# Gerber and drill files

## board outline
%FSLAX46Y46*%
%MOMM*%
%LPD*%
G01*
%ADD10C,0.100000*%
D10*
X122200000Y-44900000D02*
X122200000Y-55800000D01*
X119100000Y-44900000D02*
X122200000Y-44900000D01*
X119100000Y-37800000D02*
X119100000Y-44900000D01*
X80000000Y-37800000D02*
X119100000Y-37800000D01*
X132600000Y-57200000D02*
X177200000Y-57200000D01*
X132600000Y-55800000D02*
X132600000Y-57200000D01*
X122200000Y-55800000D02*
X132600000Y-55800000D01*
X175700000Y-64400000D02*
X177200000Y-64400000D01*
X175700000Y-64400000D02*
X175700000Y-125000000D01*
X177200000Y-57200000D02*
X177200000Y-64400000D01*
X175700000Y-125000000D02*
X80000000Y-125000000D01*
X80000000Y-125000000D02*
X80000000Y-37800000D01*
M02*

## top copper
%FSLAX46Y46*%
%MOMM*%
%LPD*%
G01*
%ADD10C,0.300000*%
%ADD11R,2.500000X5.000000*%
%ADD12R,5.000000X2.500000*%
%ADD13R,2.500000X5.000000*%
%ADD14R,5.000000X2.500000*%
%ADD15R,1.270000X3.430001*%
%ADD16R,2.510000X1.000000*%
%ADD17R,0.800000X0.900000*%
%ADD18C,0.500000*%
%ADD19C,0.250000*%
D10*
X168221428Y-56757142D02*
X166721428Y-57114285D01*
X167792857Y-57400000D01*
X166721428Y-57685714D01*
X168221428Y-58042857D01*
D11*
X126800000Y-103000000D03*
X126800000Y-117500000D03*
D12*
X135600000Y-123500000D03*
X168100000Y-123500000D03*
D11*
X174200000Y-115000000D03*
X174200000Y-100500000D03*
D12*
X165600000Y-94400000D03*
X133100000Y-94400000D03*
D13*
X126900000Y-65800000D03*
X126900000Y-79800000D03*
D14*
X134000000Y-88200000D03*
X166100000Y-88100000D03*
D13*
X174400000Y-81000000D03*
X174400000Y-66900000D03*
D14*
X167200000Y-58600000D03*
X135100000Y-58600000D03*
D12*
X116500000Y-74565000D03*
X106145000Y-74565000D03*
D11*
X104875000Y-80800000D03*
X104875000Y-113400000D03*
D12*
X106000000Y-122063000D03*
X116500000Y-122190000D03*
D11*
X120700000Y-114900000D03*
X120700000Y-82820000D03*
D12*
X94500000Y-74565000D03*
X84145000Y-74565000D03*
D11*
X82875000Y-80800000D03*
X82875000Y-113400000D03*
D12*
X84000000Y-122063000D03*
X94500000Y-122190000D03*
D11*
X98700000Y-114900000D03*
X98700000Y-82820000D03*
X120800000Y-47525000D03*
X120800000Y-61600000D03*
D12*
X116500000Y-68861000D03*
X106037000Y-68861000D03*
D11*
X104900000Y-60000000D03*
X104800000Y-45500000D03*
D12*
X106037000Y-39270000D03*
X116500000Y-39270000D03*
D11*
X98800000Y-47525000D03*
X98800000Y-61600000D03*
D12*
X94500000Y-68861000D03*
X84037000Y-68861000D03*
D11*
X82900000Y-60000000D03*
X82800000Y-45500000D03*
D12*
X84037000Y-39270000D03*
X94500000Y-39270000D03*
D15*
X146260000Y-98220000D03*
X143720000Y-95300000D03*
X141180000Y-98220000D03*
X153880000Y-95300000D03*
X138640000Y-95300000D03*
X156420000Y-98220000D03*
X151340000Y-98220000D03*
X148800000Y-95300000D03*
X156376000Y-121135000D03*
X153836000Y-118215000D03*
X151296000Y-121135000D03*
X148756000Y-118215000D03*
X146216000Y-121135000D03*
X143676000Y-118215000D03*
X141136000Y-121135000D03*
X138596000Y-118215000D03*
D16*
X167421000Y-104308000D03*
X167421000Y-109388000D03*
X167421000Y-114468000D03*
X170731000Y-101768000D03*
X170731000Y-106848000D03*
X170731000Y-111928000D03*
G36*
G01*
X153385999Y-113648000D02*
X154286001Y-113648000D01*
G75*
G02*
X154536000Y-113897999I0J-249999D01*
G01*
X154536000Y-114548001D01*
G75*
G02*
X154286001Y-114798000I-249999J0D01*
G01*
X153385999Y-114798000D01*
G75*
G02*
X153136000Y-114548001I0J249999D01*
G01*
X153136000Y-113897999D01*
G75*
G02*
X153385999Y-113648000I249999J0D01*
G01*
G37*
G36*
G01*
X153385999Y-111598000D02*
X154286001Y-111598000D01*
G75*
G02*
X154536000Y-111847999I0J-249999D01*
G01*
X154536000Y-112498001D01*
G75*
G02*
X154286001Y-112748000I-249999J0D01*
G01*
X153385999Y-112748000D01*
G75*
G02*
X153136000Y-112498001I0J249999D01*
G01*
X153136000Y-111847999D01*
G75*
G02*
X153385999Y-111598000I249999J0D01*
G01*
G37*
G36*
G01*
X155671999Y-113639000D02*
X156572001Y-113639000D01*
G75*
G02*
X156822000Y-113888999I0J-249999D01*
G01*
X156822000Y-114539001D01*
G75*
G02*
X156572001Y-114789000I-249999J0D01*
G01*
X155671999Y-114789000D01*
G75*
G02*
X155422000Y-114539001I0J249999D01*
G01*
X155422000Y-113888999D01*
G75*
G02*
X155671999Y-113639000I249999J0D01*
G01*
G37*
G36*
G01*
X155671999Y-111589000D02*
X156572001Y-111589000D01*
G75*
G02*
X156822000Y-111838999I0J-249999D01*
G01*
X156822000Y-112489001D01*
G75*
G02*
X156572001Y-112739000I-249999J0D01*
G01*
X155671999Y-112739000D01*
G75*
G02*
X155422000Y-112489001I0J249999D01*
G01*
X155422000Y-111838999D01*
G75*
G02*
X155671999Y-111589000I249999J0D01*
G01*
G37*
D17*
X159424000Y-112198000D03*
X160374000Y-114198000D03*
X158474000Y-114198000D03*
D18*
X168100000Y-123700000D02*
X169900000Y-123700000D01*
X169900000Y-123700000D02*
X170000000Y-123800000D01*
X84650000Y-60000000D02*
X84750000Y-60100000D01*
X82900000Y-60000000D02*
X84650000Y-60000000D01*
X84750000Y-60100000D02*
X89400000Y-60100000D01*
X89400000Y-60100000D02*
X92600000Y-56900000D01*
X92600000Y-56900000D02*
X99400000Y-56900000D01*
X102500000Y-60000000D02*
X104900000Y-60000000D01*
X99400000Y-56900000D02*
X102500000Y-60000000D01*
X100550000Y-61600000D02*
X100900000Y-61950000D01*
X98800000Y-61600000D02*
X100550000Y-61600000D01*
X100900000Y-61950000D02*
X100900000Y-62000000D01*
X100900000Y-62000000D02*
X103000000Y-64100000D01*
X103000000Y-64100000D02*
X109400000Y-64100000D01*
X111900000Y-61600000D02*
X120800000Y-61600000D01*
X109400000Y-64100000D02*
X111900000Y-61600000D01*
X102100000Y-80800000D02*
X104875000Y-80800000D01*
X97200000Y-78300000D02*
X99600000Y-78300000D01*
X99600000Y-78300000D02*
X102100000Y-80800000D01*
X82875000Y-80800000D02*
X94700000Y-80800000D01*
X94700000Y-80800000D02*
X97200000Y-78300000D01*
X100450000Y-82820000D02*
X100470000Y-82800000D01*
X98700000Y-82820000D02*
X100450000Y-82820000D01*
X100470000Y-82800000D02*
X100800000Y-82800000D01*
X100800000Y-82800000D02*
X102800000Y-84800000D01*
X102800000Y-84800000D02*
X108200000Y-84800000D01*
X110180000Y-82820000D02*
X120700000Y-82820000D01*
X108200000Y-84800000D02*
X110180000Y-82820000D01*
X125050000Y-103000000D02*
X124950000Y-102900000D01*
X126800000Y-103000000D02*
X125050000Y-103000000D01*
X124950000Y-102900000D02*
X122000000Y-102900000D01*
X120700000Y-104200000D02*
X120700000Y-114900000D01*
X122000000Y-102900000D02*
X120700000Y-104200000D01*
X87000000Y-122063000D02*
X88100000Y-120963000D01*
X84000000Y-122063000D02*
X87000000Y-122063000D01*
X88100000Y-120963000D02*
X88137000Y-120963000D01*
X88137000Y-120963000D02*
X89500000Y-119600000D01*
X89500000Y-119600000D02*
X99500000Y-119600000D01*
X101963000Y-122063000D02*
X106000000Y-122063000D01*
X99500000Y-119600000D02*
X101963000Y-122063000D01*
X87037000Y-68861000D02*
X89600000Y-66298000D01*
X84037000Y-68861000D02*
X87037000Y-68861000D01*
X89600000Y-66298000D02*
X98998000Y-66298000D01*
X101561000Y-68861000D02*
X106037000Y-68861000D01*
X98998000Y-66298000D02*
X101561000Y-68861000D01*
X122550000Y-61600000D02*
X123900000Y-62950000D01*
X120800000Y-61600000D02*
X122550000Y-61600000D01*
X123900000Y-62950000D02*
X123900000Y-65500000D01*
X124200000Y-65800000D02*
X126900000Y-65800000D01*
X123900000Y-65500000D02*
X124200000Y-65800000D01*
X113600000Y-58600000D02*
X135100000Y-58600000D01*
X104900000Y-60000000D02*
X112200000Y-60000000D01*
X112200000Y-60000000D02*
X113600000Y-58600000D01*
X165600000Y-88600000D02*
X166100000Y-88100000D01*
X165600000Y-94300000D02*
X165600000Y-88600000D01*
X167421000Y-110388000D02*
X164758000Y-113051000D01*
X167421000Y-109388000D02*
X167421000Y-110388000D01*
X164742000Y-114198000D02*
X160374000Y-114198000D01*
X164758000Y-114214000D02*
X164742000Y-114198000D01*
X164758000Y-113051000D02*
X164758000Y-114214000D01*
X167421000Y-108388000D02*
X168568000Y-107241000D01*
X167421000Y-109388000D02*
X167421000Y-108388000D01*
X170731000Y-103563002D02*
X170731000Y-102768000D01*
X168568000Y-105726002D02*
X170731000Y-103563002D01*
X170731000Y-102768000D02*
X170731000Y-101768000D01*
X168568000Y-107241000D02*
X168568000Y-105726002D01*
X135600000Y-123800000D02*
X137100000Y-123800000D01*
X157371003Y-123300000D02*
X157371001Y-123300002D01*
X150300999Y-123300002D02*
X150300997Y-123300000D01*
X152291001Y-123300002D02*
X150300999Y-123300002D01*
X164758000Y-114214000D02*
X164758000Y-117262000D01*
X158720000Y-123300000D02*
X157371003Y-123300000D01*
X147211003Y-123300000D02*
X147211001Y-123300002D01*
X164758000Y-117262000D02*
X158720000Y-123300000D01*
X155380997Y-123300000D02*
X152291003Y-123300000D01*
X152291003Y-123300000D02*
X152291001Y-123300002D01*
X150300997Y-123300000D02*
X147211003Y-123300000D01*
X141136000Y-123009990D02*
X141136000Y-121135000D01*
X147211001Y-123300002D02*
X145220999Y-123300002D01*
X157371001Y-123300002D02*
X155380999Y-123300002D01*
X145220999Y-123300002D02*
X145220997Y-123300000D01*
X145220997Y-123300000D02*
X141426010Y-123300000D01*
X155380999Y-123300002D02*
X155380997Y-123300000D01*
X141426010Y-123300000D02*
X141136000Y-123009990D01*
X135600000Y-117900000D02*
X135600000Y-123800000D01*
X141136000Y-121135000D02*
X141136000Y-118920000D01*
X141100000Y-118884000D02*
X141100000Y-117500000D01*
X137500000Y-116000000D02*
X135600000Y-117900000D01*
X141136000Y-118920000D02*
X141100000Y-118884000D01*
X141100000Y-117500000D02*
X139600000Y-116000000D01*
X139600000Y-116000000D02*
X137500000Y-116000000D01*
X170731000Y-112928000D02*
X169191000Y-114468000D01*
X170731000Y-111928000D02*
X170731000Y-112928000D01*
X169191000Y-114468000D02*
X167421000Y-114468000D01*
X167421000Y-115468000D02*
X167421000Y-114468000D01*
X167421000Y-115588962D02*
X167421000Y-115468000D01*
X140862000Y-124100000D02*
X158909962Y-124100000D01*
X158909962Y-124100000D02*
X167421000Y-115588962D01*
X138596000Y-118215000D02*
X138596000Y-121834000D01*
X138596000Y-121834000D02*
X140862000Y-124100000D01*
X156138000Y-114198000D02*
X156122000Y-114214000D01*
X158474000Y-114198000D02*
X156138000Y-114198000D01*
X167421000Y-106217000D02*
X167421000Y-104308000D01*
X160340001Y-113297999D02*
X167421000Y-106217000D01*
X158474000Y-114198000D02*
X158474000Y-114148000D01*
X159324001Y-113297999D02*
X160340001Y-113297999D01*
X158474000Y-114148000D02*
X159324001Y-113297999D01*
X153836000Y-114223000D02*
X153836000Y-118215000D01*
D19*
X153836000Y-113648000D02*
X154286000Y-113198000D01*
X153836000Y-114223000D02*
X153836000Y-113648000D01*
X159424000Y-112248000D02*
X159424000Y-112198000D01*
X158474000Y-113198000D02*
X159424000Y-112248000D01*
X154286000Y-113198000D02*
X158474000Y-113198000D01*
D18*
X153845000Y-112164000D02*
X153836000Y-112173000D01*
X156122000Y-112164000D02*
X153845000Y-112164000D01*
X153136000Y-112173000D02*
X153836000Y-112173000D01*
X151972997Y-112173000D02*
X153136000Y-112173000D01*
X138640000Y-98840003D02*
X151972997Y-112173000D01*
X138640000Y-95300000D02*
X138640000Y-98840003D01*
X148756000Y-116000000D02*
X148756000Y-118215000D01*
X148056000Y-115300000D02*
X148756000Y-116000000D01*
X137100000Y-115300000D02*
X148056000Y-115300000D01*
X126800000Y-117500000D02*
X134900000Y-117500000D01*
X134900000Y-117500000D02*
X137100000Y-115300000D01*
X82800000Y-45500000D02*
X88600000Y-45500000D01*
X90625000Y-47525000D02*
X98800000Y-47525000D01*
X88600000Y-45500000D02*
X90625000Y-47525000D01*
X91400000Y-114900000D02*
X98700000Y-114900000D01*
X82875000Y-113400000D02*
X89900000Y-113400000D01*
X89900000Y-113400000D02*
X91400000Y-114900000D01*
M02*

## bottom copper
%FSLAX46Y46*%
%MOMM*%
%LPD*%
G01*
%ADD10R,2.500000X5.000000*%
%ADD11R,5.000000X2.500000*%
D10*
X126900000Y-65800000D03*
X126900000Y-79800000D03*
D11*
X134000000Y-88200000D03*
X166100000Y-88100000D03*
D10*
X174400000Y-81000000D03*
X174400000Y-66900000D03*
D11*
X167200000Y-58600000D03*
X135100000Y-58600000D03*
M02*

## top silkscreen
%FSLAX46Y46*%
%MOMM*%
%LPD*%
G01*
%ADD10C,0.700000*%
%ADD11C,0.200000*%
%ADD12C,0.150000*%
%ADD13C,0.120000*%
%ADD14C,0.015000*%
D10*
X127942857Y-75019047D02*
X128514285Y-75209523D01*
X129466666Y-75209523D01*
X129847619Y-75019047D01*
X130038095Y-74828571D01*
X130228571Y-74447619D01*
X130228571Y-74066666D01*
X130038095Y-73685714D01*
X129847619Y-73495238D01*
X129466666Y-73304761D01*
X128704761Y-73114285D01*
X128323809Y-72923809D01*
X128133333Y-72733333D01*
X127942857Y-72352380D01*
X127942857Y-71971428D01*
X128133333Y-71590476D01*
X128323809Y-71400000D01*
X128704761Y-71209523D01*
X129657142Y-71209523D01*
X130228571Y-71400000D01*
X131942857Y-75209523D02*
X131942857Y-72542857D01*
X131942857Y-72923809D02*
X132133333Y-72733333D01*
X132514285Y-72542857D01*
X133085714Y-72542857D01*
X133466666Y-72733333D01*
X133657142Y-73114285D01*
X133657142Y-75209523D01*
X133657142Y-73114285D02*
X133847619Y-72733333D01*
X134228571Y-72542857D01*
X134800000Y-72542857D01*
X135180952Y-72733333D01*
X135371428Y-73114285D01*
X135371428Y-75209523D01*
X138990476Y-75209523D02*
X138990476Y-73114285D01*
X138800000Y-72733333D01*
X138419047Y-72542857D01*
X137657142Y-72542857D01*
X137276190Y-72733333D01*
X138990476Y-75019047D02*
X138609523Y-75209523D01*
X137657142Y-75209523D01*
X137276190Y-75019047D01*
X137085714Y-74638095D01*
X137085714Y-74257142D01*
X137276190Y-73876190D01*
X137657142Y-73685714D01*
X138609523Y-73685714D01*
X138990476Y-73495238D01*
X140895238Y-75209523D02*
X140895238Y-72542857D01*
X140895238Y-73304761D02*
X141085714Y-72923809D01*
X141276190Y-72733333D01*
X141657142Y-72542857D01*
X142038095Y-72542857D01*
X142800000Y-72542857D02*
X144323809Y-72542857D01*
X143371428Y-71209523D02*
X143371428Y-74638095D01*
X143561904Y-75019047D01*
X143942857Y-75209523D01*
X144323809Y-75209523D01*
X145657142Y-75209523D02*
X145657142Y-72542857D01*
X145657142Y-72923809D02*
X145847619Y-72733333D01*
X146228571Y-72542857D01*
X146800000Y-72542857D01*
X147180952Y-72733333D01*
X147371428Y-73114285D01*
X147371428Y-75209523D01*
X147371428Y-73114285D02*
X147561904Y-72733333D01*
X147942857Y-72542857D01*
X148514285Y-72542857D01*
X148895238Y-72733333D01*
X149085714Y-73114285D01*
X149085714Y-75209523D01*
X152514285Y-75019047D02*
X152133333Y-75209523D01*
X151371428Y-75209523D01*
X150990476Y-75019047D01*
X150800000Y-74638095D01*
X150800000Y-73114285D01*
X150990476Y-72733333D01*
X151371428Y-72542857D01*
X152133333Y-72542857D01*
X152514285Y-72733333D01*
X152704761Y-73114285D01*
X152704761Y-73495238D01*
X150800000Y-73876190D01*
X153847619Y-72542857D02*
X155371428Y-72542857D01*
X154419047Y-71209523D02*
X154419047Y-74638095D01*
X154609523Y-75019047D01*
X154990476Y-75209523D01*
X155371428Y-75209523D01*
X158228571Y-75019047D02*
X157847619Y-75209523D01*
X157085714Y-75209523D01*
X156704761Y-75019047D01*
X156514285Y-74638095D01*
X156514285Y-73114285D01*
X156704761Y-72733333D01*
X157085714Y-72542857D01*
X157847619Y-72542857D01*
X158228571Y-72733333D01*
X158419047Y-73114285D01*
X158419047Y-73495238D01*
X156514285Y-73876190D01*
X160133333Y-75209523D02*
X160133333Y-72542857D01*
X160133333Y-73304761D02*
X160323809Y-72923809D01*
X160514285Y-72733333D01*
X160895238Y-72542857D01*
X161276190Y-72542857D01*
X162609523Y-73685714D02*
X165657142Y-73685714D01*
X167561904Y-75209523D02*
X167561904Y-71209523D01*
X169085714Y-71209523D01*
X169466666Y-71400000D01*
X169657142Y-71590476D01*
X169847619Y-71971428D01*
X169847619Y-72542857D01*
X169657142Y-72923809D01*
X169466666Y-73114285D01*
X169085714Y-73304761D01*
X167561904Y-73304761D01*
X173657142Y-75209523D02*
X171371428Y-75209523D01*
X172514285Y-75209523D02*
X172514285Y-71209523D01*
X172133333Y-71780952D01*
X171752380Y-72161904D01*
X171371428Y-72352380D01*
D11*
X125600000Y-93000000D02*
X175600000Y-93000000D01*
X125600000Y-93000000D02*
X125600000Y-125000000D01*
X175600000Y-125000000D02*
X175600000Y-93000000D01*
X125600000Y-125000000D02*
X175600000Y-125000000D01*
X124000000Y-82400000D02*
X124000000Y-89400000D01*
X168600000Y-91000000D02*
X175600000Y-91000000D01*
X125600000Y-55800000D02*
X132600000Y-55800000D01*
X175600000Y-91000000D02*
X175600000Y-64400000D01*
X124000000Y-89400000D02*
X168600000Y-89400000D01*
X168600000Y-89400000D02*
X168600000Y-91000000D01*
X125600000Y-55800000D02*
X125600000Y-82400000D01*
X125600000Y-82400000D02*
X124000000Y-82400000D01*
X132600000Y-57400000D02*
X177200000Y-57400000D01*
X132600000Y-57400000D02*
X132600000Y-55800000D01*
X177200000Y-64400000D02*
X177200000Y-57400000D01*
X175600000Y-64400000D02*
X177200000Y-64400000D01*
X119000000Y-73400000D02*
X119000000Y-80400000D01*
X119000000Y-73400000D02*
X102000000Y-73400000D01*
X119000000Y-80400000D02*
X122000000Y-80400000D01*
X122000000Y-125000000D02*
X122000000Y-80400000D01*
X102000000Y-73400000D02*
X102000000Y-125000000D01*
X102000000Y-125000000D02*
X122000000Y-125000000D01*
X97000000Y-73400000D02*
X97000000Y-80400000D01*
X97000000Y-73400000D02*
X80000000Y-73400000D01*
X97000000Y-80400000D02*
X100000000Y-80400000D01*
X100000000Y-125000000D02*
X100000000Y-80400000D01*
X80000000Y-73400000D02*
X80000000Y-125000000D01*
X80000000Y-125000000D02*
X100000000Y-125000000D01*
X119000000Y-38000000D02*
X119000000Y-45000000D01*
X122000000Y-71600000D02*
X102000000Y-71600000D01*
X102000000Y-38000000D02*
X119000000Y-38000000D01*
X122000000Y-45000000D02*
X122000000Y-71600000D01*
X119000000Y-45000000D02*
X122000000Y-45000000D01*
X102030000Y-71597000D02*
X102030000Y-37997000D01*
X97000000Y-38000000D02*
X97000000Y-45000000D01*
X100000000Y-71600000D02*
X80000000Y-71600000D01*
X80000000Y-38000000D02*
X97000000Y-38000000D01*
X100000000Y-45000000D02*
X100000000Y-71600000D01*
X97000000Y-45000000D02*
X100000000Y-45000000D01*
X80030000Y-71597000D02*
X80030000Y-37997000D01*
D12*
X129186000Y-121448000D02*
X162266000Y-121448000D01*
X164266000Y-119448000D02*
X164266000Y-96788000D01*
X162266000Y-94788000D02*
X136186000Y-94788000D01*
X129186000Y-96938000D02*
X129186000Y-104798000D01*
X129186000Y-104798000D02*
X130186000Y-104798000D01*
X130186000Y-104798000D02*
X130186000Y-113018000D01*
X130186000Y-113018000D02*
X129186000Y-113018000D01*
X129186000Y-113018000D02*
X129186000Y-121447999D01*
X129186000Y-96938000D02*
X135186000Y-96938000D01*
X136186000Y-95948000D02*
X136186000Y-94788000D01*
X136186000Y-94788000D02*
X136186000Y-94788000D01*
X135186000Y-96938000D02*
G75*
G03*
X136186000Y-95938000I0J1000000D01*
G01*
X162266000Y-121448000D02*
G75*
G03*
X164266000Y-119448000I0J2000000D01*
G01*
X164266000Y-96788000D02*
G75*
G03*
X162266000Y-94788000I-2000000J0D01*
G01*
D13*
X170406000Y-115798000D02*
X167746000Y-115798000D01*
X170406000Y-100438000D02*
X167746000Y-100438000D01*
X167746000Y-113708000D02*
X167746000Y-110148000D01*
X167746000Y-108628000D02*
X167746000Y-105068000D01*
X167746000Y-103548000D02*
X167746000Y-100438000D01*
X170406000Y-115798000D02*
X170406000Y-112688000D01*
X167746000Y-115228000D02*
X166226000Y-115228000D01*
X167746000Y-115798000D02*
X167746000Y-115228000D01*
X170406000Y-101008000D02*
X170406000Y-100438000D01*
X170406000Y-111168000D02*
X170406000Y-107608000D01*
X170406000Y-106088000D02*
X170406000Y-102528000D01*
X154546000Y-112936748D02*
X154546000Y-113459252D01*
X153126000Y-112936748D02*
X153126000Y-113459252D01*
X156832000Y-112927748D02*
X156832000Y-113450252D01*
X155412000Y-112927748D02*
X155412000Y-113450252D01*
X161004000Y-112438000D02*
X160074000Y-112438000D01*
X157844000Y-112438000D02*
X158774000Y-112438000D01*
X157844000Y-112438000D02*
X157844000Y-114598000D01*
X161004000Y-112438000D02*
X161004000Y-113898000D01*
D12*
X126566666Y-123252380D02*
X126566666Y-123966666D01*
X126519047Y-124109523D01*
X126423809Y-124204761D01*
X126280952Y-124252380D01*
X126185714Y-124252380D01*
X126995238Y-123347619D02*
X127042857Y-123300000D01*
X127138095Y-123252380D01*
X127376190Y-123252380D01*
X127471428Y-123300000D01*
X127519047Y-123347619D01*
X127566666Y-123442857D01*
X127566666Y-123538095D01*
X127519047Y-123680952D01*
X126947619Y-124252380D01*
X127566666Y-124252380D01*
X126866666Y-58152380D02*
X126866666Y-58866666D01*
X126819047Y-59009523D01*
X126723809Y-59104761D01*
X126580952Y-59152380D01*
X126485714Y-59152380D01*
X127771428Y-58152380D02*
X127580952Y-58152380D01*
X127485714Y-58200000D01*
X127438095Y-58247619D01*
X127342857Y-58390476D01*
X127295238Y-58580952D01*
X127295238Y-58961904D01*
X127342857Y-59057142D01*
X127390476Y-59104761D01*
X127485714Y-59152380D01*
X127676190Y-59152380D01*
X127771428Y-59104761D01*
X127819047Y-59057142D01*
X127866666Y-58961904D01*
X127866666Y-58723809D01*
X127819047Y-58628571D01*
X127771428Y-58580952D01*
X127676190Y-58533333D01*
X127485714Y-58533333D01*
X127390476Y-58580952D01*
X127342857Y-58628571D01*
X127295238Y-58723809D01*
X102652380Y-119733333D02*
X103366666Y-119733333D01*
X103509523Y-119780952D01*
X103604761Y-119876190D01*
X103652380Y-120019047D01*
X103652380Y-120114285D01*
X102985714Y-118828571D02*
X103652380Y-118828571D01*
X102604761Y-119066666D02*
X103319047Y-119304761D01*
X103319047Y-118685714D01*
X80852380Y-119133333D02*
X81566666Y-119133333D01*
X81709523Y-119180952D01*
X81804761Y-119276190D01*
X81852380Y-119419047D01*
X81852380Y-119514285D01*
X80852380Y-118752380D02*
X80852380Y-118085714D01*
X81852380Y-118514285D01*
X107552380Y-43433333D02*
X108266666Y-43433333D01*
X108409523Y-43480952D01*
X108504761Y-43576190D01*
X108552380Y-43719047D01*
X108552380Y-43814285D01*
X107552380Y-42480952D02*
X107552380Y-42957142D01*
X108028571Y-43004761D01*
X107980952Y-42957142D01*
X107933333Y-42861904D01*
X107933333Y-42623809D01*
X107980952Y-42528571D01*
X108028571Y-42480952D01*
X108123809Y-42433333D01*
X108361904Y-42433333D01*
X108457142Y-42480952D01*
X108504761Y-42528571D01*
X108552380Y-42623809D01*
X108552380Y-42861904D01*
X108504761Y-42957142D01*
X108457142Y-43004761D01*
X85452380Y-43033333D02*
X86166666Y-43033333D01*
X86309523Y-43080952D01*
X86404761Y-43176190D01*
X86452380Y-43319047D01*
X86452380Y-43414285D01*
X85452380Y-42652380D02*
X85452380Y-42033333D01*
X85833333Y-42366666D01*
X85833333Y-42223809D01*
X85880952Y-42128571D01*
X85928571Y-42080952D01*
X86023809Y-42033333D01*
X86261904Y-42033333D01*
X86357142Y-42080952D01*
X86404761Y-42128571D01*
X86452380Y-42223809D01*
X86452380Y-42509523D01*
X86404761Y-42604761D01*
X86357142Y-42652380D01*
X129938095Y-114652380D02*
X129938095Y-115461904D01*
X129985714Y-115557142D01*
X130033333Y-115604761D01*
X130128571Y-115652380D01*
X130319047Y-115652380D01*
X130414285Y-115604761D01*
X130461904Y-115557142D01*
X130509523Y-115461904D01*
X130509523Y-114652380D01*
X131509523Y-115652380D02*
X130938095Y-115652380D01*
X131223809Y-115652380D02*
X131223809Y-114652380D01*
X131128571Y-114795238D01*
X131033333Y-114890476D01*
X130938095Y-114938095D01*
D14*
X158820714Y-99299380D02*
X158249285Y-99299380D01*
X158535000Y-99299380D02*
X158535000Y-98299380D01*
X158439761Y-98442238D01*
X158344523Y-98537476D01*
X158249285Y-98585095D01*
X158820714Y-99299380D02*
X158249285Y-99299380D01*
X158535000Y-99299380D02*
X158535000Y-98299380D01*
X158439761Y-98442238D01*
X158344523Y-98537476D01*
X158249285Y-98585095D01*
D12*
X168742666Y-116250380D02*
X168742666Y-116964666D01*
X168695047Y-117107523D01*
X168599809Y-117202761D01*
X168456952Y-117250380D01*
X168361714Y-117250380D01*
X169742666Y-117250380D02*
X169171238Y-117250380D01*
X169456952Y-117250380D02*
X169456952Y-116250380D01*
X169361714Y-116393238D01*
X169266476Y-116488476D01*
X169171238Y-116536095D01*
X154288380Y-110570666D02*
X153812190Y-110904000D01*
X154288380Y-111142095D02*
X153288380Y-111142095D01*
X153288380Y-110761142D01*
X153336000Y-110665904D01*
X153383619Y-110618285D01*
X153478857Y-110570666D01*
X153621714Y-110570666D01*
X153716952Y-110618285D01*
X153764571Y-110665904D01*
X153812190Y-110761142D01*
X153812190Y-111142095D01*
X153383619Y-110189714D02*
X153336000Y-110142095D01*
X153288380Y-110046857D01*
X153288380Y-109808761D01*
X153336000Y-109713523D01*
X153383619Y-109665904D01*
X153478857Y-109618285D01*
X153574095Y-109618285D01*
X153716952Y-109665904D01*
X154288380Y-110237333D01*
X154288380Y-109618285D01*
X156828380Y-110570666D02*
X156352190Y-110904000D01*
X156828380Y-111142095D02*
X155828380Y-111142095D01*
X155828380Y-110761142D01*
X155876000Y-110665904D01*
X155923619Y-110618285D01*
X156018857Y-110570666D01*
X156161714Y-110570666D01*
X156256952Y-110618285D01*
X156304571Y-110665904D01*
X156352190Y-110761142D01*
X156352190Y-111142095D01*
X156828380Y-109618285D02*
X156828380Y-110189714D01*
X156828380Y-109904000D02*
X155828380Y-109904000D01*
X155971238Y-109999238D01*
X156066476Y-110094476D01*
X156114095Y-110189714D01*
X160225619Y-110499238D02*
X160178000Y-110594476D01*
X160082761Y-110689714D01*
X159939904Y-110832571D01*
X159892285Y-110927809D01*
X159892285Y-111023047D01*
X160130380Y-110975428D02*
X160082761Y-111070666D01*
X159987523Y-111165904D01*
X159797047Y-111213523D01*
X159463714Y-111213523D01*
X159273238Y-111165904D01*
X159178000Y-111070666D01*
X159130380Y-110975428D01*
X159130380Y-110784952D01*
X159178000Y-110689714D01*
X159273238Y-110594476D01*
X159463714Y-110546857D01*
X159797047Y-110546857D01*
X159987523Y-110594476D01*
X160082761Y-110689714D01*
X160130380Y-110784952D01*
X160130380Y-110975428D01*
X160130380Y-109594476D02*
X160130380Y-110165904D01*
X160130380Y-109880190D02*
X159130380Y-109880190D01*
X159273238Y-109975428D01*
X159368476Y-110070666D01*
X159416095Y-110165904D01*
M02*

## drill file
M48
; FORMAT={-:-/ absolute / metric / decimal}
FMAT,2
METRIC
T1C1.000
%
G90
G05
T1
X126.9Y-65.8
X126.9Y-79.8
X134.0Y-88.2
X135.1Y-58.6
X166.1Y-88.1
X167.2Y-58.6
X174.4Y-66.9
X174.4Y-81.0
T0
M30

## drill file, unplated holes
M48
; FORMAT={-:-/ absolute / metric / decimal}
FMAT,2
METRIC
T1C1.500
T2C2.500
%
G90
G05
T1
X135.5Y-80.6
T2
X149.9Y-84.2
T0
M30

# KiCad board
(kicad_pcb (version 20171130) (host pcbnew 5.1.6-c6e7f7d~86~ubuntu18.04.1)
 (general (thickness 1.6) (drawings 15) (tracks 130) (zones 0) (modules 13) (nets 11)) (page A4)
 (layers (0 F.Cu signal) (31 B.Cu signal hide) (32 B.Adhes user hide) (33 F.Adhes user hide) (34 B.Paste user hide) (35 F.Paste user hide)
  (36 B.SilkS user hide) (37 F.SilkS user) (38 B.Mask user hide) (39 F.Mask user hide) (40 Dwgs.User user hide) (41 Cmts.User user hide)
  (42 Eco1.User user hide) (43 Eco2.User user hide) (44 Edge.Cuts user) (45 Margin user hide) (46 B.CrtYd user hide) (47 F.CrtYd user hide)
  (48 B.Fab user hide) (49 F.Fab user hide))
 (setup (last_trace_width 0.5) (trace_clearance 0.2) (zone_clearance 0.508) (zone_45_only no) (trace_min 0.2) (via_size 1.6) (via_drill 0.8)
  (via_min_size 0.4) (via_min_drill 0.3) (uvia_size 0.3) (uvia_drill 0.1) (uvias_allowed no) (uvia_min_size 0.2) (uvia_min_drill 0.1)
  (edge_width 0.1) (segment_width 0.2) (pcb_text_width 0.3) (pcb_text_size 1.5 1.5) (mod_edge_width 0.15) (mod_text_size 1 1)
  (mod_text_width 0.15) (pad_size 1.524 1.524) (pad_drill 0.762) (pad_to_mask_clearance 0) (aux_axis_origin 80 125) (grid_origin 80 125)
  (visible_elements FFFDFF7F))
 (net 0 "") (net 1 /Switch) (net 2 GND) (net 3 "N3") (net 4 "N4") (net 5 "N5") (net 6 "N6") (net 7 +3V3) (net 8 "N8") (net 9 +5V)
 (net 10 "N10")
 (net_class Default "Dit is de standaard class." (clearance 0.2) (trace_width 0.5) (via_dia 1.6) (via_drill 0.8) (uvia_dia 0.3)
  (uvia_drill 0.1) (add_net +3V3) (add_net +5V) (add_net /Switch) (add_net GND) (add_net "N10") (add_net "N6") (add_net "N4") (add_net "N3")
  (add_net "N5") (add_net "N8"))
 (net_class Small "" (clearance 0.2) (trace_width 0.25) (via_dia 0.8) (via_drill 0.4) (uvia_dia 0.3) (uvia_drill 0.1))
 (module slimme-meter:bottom (layer F.Cu) (at 125.6 125)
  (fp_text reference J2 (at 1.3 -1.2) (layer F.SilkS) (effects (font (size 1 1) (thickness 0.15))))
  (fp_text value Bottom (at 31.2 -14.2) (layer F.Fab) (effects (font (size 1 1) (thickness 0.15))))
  (fp_line (start 0 -32) (end 50 -32) (layer F.SilkS) (width 0.2))
  (fp_line (start 0 -32) (end 0 0) (layer F.SilkS) (width 0.2))
  (fp_line (start 50 0) (end 50 -32) (layer F.SilkS) (width 0.2)) (fp_line (start 0 0) (end 50 0) (layer F.SilkS) (width 0.2))
  (pad 8 smd rect (at 1.2 -22 270) (size 5 2.5) (layers F.Cu F.Paste F.Mask))
  (pad 7 smd rect (at 1.2 -7.5 270) (size 5 2.5) (layers F.Cu F.Paste F.Mask) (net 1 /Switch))
  (pad 6 smd rect (at 10 -1.5) (size 5 2.5) (layers F.Cu F.Paste F.Mask) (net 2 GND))
  (pad 5 smd rect (at 42.5 -1.5 180) (size 5 2.5) (layers F.Cu F.Paste F.Mask))
  (pad 4 smd rect (at 48.6 -10 90) (size 5 2.5) (layers F.Cu F.Paste F.Mask))
  (pad 3 smd rect (at 48.6 -24.5 90) (size 5 2.5) (layers F.Cu F.Paste F.Mask))
  (pad 2 smd rect (at 40 -30.6) (size 5 2.5) (layers F.Cu F.Paste F.Mask))
  (pad 1 smd rect (at 7.5 -30.6) (size 5 2.5) (layers F.Cu F.Paste F.Mask)))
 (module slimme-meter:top (layer F.Cu) (at 125.6 57.4)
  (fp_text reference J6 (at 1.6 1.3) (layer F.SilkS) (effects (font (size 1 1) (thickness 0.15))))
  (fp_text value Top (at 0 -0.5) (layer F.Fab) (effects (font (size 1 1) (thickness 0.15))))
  (fp_line (start -1.6 25) (end -1.6 32) (layer F.SilkS) (width 0.2))
  (fp_line (start 43 33.6) (end 50 33.6) (layer F.SilkS) (width 0.2))
  (fp_line (start 0 -1.6) (end 7 -1.6) (layer F.SilkS) (width 0.2))
  (fp_line (start 50 33.6) (end 50 7) (layer F.SilkS) (width 0.2))
  (fp_line (start -1.6 32) (end 43 32) (layer F.SilkS) (width 0.2))
  (fp_line (start 43 32) (end 43 33.6) (layer F.SilkS) (width 0.2))
  (fp_line (start 0 -1.6) (end 0 25) (layer F.SilkS) (width 0.2))
  (fp_line (start 0 25) (end -1.6 25) (layer F.SilkS) (width 0.2))
  (fp_line (start 7 0) (end 51.6 0) (layer F.SilkS) (width 0.2))
  (fp_line (start 7 0) (end 7 -1.6) (layer F.SilkS) (width 0.2))
  (fp_line (start 51.6 7) (end 51.6 0) (layer F.SilkS) (width 0.2))
  (fp_line (start 50 7) (end 51.6 7) (layer F.SilkS) (width 0.2))
  (pad 8 thru_hole rect (at 1.3 8.4 270) (size 5 2.5) (drill 1) (layers *.Cu *.Mask))
  (pad 7 thru_hole rect (at 1.3 22.4 270) (size 5 2.5) (drill 1) (layers *.Cu *.Mask) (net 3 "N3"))
  (pad 6 thru_hole rect (at 8.4 30.8 180) (size 5 2.5) (drill 1) (layers *.Cu *.Mask) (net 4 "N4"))
  (pad 5 thru_hole rect (at 40.5 30.7 180) (size 5 2.5) (drill 1) (layers *.Cu *.Mask))
  (pad 4 thru_hole rect (at 48.8 23.6 90) (size 5 2.5) (drill 1) (layers *.Cu *.Mask))
  (pad 3 thru_hole rect (at 48.8 9.5 90) (size 5 2.5) (drill 1) (layers *.Cu *.Mask))
  (pad 2 thru_hole rect (at 41.6 1.2) (size 5 2.5) (drill 1) (layers *.Cu *.Mask))
  (pad 1 thru_hole rect (at 9.5 1.2) (size 5 2.5) (drill 1) (layers *.Cu *.Mask)))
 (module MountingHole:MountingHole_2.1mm (layer F.Cu) (at 135.5 80.6)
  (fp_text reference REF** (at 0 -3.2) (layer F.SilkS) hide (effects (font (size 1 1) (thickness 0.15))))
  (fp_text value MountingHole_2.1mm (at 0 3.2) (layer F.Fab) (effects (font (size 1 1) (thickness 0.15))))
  (pad "" np_thru_hole circle (at 0 0) (size 1.5 1.5) (drill 1.5) (layers *.Cu *.Mask)))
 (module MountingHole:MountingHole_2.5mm (layer F.Cu) (at 149.9 84.2)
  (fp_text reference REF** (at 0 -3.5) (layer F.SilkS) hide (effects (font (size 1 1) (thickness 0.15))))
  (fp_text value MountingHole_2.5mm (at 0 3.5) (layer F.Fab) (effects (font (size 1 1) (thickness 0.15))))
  (pad 1 np_thru_hole circle (at 0 0) (size 2.5 2.5) (drill 2.5) (layers *.Cu *.Mask)))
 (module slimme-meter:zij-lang (layer F.Cu) (at 102 125 270)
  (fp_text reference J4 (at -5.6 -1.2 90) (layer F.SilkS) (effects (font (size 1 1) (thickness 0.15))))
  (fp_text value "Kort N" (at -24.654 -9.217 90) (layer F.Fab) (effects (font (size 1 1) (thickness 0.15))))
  (fp_line (start -51.6 -17) (end -44.6 -17) (layer F.SilkS) (width 0.2))
  (fp_line (start -51.6 -17) (end -51.6 0) (layer F.SilkS) (width 0.2))
  (fp_line (start -44.6 -17) (end -44.6 -20) (layer F.SilkS) (width 0.2))
  (fp_line (start 0 -20) (end -44.6 -20) (layer F.SilkS) (width 0.2))
  (fp_line (start -51.6 0) (end 0 0) (layer F.SilkS) (width 0.2))
  (fp_line (start 0 0) (end 0 -20) (layer F.SilkS) (width 0.2))
  (pad 8 smd rect (at -50.435 -14.5 180) (size 5 2.5) (layers F.Cu F.Paste F.Mask))
  (pad 7 smd rect (at -50.435 -4.145 180) (size 5 2.5) (layers F.Cu F.Paste F.Mask))
  (pad 6 smd rect (at -44.2 -2.875 270) (size 5 2.5) (layers F.Cu F.Paste F.Mask))
  (pad 5 smd rect (at -11.6 -2.875 90) (size 5 2.5) (layers F.Cu F.Paste F.Mask))
  (pad 4 smd rect (at -2.937 -4) (size 5 2.5) (layers F.Cu F.Paste F.Mask))
  (pad 3 smd rect (at -2.81 -14.5) (size 5 2.5) (layers F.Cu F.Paste F.Mask))
  (pad 2 smd rect (at -10.1 -18.7 270) (size 5 2.5) (layers F.Cu F.Paste F.Mask))
  (pad 1 smd rect (at -42.18 -18.7 270) (size 5 2.5) (layers F.Cu F.Paste F.Mask)))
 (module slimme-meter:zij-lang (layer F.Cu) (at 80 125 270)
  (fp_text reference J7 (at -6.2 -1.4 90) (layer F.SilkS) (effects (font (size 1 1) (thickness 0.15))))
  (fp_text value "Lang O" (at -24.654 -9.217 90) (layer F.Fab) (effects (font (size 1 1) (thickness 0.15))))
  (fp_line (start -51.6 -17) (end -44.6 -17) (layer F.SilkS) (width 0.2))
  (fp_line (start -51.6 -17) (end -51.6 0) (layer F.SilkS) (width 0.2))
  (fp_line (start -44.6 -17) (end -44.6 -20) (layer F.SilkS) (width 0.2))
  (fp_line (start 0 -20) (end -44.6 -20) (layer F.SilkS) (width 0.2))
  (fp_line (start -51.6 0) (end 0 0) (layer F.SilkS) (width 0.2))
  (fp_line (start 0 0) (end 0 -20) (layer F.SilkS) (width 0.2))
  (pad 8 smd rect (at -50.435 -14.5 180) (size 5 2.5) (layers F.Cu F.Paste F.Mask))
  (pad 7 smd rect (at -50.435 -4.145 180) (size 5 2.5) (layers F.Cu F.Paste F.Mask))
  (pad 6 smd rect (at -44.2 -2.875 270) (size 5 2.5) (layers F.Cu F.Paste F.Mask))
  (pad 5 smd rect (at -11.6 -2.875 90) (size 5 2.5) (layers F.Cu F.Paste F.Mask) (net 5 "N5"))
  (pad 4 smd rect (at -2.937 -4) (size 5 2.5) (layers F.Cu F.Paste F.Mask))
  (pad 3 smd rect (at -2.81 -14.5) (size 5 2.5) (layers F.Cu F.Paste F.Mask))
  (pad 2 smd rect (at -10.1 -18.7 270) (size 5 2.5) (layers F.Cu F.Paste F.Mask) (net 5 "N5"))
  (pad 1 smd rect (at -42.18 -18.7 270) (size 5 2.5) (layers F.Cu F.Paste F.Mask)))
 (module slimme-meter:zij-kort (layer F.Cu) (at 102 38 180)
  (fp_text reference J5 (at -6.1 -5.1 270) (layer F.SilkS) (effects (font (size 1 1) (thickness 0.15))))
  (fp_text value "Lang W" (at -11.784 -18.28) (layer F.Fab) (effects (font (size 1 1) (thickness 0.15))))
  (fp_line (start -17 0) (end -17 -7) (layer F.SilkS) (width 0.2))
  (fp_line (start -20 -33.6) (end 0 -33.6) (layer F.SilkS) (width 0.2))
  (fp_line (start 0 0) (end -17 0) (layer F.SilkS) (width 0.2))
  (fp_line (start -20 -7) (end -20 -33.6) (layer F.SilkS) (width 0.2))
  (fp_line (start -17 -7) (end -20 -7) (layer F.SilkS) (width 0.2))
  (fp_line (start -0.03 -33.597) (end -0.03 0.003) (layer F.SilkS) (width 0.2))
  (pad 8 smd rect (at -18.8 -9.525 90) (size 5 2.5) (layers F.Cu F.Paste F.Mask))
  (pad 7 smd rect (at -18.8 -23.6 90) (size 5 2.5) (layers F.Cu F.Paste F.Mask))
  (pad 6 smd rect (at -14.5 -30.861) (size 5 2.5) (layers F.Cu F.Paste F.Mask))
  (pad 5 smd rect (at -4.037 -30.861) (size 5 2.5) (layers F.Cu F.Paste F.Mask))
  (pad 4 smd rect (at -2.9 -22 270) (size 5 2.5) (layers F.Cu F.Paste F.Mask))
  (pad 3 smd rect (at -2.8 -7.5 270) (size 5 2.5) (layers F.Cu F.Paste F.Mask))
  (pad 2 smd rect (at -4.037 -1.27 180) (size 5 2.5) (layers F.Cu F.Paste F.Mask))
  (pad 1 smd rect (at -14.5 -1.27 180) (size 5 2.5) (layers F.Cu F.Paste F.Mask)))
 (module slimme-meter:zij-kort (layer F.Cu) (at 80 38 180)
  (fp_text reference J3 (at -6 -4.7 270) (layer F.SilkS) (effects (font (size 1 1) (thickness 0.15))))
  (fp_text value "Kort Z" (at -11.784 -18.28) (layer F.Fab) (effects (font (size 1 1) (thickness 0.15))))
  (fp_line (start -17 0) (end -17 -7) (layer F.SilkS) (width 0.2))
  (fp_line (start -20 -33.6) (end 0 -33.6) (layer F.SilkS) (width 0.2))
  (fp_line (start 0 0) (end -17 0) (layer F.SilkS) (width 0.2))
  (fp_line (start -20 -7) (end -20 -33.6) (layer F.SilkS) (width 0.2))
  (fp_line (start -17 -7) (end -20 -7) (layer F.SilkS) (width 0.2))
  (fp_line (start -0.03 -33.597) (end -0.03 0.003) (layer F.SilkS) (width 0.2))
  (pad 8 smd rect (at -18.8 -9.525 90) (size 5 2.5) (layers F.Cu F.Paste F.Mask) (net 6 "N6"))
  (pad 7 smd rect (at -18.8 -23.6 90) (size 5 2.5) (layers F.Cu F.Paste F.Mask))
  (pad 6 smd rect (at -14.5 -30.861) (size 5 2.5) (layers F.Cu F.Paste F.Mask))
  (pad 5 smd rect (at -4.037 -30.861) (size 5 2.5) (layers F.Cu F.Paste F.Mask))
  (pad 4 smd rect (at -2.9 -22 270) (size 5 2.5) (layers F.Cu F.Paste F.Mask))
  (pad 3 smd rect (at -2.8 -7.5 270) (size 5 2.5) (layers F.Cu F.Paste F.Mask) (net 6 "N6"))
  (pad 2 smd rect (at -4.037 -1.27 180) (size 5 2.5) (layers F.Cu F.Paste F.Mask))
  (pad 1 smd rect (at -14.5 -1.27 180) (size 5 2.5) (layers F.Cu F.Paste F.Mask)))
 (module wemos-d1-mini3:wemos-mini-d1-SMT (layer F.Cu) (at 147.486 108.118)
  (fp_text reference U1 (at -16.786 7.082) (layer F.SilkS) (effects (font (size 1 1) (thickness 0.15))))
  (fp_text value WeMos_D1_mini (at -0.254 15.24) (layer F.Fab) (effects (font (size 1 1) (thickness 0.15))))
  (fp_line (start -18.3 13.33) (end 14.78 13.33) (layer F.SilkS) (width 0.15))
  (fp_line (start 16.78 11.33) (end 16.78 -11.33) (layer F.SilkS) (width 0.15))
  (fp_line (start 14.78 -13.33) (end -11.3 -13.33) (layer F.SilkS) (width 0.15))
  (fp_line (start -18.3 -11.18) (end -18.3 -3.32) (layer F.SilkS) (width 0.15))
  (fp_line (start -18.3 -3.32) (end -17.3 -3.32) (layer F.SilkS) (width 0.15))
  (fp_line (start -17.3 -3.32) (end -17.3 4.9) (layer F.SilkS) (width 0.15))
  (fp_line (start -17.3 4.9) (end -18.3 4.9) (layer F.SilkS) (width 0.15))
  (fp_line (start -18.3 4.9) (end -18.3 13.329999) (layer F.SilkS) (width 0.15))
  (fp_line (start -18.3 -11.18) (end -12.3 -11.18) (layer F.SilkS) (width 0.15))
  (fp_line (start -11.3 -12.17) (end -11.3 -13.33) (layer F.SilkS) (width 0.15))
  (fp_line (start -11.3 -13.33) (end -11.3 -13.33) (layer F.SilkS) (width 0.15))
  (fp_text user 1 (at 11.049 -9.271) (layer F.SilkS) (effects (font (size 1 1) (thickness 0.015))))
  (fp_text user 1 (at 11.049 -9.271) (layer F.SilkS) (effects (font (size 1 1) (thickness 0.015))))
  (fp_arc (start -12.3 -12.18) (end -11.3 -12.18) (angle 90) (layer F.SilkS) (width 0.15))
  (fp_arc (start 14.78 11.33) (end 16.78 11.33) (angle 90) (layer F.SilkS) (width 0.15))
  (fp_arc (start 14.78 -11.33) (end 14.78 -13.33) (angle 90) (layer F.SilkS) (width 0.15))
  (pad 5 smd rect (at -1.226 -9.898 180) (size 1.27 3.430001) (layers F.Cu F.Paste))
  (pad 6 smd rect (at -3.766 -12.818 180) (size 1.27 3.430001) (layers F.Cu F.Paste))
  (pad 7 smd rect (at -6.306 -9.898 180) (size 1.27 3.430001) (layers F.Cu F.Paste))
  (pad 2 smd rect (at 6.394 -12.818 180) (size 1.27 3.430001) (layers F.Cu F.Paste))
  (pad 8 smd rect (at -8.846 -12.818 180) (size 1.27 3.430001) (layers F.Cu F.Paste) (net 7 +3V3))
  (pad 1 smd rect (at 8.934 -9.898 180) (size 1.27 3.430001) (layers F.Cu F.Paste))
  (pad 3 smd rect (at 3.854 -9.898 180) (size 1.27 3.430001) (layers F.Cu F.Paste))
  (pad 4 smd rect (at 1.314 -12.818 180) (size 1.27 3.430001) (layers F.Cu F.Paste))
  (pad 16 smd rect (at 8.89 13.017) (size 1.27 3.430001) (layers F.Cu F.Paste))
  (pad 15 smd rect (at 6.35 10.097) (size 1.27 3.430001) (layers F.Cu F.Paste) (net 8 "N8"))
  (pad 14 smd rect (at 3.81 13.017) (size 1.27 3.430001) (layers F.Cu F.Paste))
  (pad 13 smd rect (at 1.27 10.097) (size 1.27 3.430001) (layers F.Cu F.Paste) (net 1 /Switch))
  (pad 12 smd rect (at -1.27 13.017) (size 1.27 3.430001) (layers F.Cu F.Paste))
  (pad 11 smd rect (at -3.81 10.097) (size 1.27 3.430001) (layers F.Cu F.Paste))
  (pad 10 smd rect (at -6.35 13.017) (size 1.27 3.430001) (layers F.Cu F.Paste) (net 2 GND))
  (pad 9 smd rect (at -8.89 10.097) (size 1.27 3.430001) (layers F.Cu F.Paste) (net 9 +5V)))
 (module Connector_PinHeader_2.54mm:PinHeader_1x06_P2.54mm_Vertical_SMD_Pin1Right (layer F.Cu) (at 169.076 108.118 180)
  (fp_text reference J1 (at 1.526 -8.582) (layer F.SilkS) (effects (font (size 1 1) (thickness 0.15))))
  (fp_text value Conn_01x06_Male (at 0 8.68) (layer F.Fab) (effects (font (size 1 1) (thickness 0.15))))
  (fp_line (start -1.33 -7.68) (end 1.33 -7.68) (layer F.SilkS) (width 0.12))
  (fp_line (start -1.33 7.68) (end 1.33 7.68) (layer F.SilkS) (width 0.12))
  (fp_line (start 1.33 -5.59) (end 1.33 -2.03) (layer F.SilkS) (width 0.12))
  (fp_line (start 1.33 -0.51) (end 1.33 3.05) (layer F.SilkS) (width 0.12))
  (fp_line (start 1.33 4.57) (end 1.33 7.68) (layer F.SilkS) (width 0.12))
  (fp_line (start -1.33 -7.68) (end -1.33 -4.57) (layer F.SilkS) (width 0.12))
  (fp_line (start 1.33 -7.11) (end 2.85 -7.11) (layer F.SilkS) (width 0.12))
  (fp_line (start 1.33 -7.68) (end 1.33 -7.11) (layer F.SilkS) (width 0.12))
  (fp_line (start -1.33 7.11) (end -1.33 7.68) (layer F.SilkS) (width 0.12))
  (fp_line (start -1.33 -3.05) (end -1.33 0.51) (layer F.SilkS) (width 0.12))
  (fp_line (start -1.33 2.03) (end -1.33 5.59) (layer F.SilkS) (width 0.12))
  (pad 5 smd rect (at 1.655 3.81 180) (size 2.51 1) (layers F.Cu F.Paste F.Mask) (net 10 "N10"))
  (pad 3 smd rect (at 1.655 -1.27 180) (size 2.51 1) (layers F.Cu F.Paste F.Mask) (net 2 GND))
  (pad 1 smd rect (at 1.655 -6.35 180) (size 2.51 1) (layers F.Cu F.Paste F.Mask) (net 9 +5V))
  (pad 6 smd rect (at -1.655 6.35 180) (size 2.51 1) (layers F.Cu F.Paste F.Mask) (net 2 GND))
  (pad 4 smd rect (at -1.655 1.27 180) (size 2.51 1) (layers F.Cu F.Paste F.Mask))
  (pad 2 smd rect (at -1.655 -3.81 180) (size 2.51 1) (layers F.Cu F.Paste F.Mask) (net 9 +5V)))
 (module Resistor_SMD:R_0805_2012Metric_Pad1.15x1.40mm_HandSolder (layer F.Cu) (at 153.836 113.198 270)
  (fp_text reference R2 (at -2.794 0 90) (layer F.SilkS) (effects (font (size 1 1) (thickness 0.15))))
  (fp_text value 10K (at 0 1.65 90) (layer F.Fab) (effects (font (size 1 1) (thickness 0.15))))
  (fp_line (start -0.261252 -0.71) (end 0.261252 -0.71) (layer F.SilkS) (width 0.12))
  (fp_line (start -0.261252 0.71) (end 0.261252 0.71) (layer F.SilkS) (width 0.12))
  (pad 2 smd roundrect (at 1.025 0 270) (size 1.15 1.4) (layers F.Cu F.Paste F.Mask) (roundrect_rratio 0.217391) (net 8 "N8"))
  (pad 1 smd roundrect (at -1.025 0 270) (size 1.15 1.4) (layers F.Cu F.Paste F.Mask) (roundrect_rratio 0.217391) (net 7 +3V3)))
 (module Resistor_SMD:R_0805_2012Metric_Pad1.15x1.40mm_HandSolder (layer F.Cu) (at 156.122 113.189 270)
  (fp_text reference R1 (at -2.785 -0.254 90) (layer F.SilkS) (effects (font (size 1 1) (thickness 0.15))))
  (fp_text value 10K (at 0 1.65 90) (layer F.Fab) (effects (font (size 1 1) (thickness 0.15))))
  (fp_line (start -0.261252 -0.71) (end 0.261252 -0.71) (layer F.SilkS) (width 0.12))
  (fp_line (start -0.261252 0.71) (end 0.261252 0.71) (layer F.SilkS) (width 0.12))
  (pad 2 smd roundrect (at 1.025 0 270) (size 1.15 1.4) (layers F.Cu F.Paste F.Mask) (roundrect_rratio 0.217391) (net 10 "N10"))
  (pad 1 smd roundrect (at -1.025 0 270) (size 1.15 1.4) (layers F.Cu F.Paste F.Mask) (roundrect_rratio 0.217391) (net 7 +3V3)))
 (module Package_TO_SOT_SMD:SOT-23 (layer F.Cu) (at 159.424 113.198 90)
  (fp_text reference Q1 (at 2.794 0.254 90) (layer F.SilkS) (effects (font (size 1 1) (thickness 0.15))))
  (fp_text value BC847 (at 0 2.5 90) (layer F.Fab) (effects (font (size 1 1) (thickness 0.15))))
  (fp_line (start 0.76 1.58) (end 0.76 0.65) (layer F.SilkS) (width 0.12))
  (fp_line (start 0.76 -1.58) (end 0.76 -0.65) (layer F.SilkS) (width 0.12))
  (fp_line (start 0.76 -1.58) (end -1.4 -1.58) (layer F.SilkS) (width 0.12))
  (fp_line (start 0.76 1.58) (end -0.7 1.58) (layer F.SilkS) (width 0.12))
  (pad 3 smd rect (at 1 0 90) (size 0.9 0.8) (layers F.Cu F.Paste F.Mask) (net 8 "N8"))
  (pad 2 smd rect (at -1 0.95 90) (size 0.9 0.8) (layers F.Cu F.Paste F.Mask) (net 2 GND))
  (pad 1 smd rect (at -1 -0.95 90) (size 0.9 0.8) (layers F.Cu F.Paste F.Mask) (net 10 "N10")))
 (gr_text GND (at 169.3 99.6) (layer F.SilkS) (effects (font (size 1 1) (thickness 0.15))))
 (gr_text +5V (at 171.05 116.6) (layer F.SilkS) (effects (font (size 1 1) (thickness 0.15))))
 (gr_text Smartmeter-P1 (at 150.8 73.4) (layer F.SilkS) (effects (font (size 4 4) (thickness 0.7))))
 (gr_line (start 122.2 44.9) (end 122.2 55.8) (layer Edge.Cuts) (width 0.1))
 (gr_line (start 119.1 44.9) (end 122.2 44.9) (layer Edge.Cuts) (width 0.1))
 (gr_line (start 119.1 37.8) (end 119.1 44.9) (layer Edge.Cuts) (width 0.1))
 (gr_line (start 80 37.8) (end 119.1 37.8) (layer Edge.Cuts) (width 0.1))
 (gr_line (start 132.6 57.2) (end 177.2 57.2) (layer Edge.Cuts) (width 0.1))
 (gr_line (start 132.6 55.8) (end 132.6 57.2) (layer Edge.Cuts) (width 0.1))
 (gr_line (start 122.2 55.8) (end 132.6 55.8) (layer Edge.Cuts) (width 0.1))
 (gr_line (start 175.7 64.4) (end 177.2 64.4) (layer Edge.Cuts) (width 0.1))
 (gr_line (start 175.7 64.4) (end 175.7 125) (layer Edge.Cuts) (width 0.1))
 (gr_line (start 177.2 57.2) (end 177.2 64.4) (layer Edge.Cuts) (width 0.1))
 (gr_line (start 175.7 125) (end 80 125) (layer Edge.Cuts) (width 0.1))
 (gr_line (start 80 125) (end 80 37.8) (layer Edge.Cuts) (width 0.1))
 (segment (start 168.1 123.7) (end 169.9 123.7) (width 0.5) (layer F.Cu) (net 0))
 (segment (start 169.9 123.7) (end 170 123.8) (width 0.5) (layer F.Cu) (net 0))
 (segment (start 84.65 60) (end 84.75 60.1) (width 0.5) (layer F.Cu) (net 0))
 (segment (start 82.9 60) (end 84.65 60) (width 0.5) (layer F.Cu) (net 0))
 (segment (start 84.75 60.1) (end 89.4 60.1) (width 0.5) (layer F.Cu) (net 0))
 (segment (start 89.4 60.1) (end 92.6 56.9) (width 0.5) (layer F.Cu) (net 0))
 (segment (start 92.6 56.9) (end 99.4 56.9) (width 0.5) (layer F.Cu) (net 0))
 (segment (start 102.5 60) (end 104.9 60) (width 0.5) (layer F.Cu) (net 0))
 (segment (start 99.4 56.9) (end 102.5 60) (width 0.5) (layer F.Cu) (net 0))
 (segment (start 100.55 61.6) (end 100.9 61.95) (width 0.5) (layer F.Cu) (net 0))
 (segment (start 98.8 61.6) (end 100.55 61.6) (width 0.5) (layer F.Cu) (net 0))
 (segment (start 100.9 61.95) (end 100.9 62) (width 0.5) (layer F.Cu) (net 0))
 (segment (start 100.9 62) (end 103 64.1) (width 0.5) (layer F.Cu) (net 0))
 (segment (start 103 64.1) (end 109.4 64.1) (width 0.5) (layer F.Cu) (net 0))
 (segment (start 111.9 61.6) (end 120.8 61.6) (width 0.5) (layer F.Cu) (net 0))
 (segment (start 109.4 64.1) (end 111.9 61.6) (width 0.5) (layer F.Cu) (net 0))
 (segment (start 102.1 80.8) (end 104.875 80.8) (width 0.5) (layer F.Cu) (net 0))
 (segment (start 97.2 78.3) (end 99.6 78.3) (width 0.5) (layer F.Cu) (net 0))
 (segment (start 99.6 78.3) (end 102.1 80.8) (width 0.5) (layer F.Cu) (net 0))
 (segment (start 82.875 80.8) (end 94.7 80.8) (width 0.5) (layer F.Cu) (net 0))
 (segment (start 94.7 80.8) (end 97.2 78.3) (width 0.5) (layer F.Cu) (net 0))
 (segment (start 100.45 82.82) (end 100.47 82.8) (width 0.5) (layer F.Cu) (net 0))
 (segment (start 98.7 82.82) (end 100.45 82.82) (width 0.5) (layer F.Cu) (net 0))
 (segment (start 100.47 82.8) (end 100.8 82.8) (width 0.5) (layer F.Cu) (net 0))
 (segment (start 100.8 82.8) (end 102.8 84.8) (width 0.5) (layer F.Cu) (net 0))
 (segment (start 102.8 84.8) (end 108.2 84.8) (width 0.5) (layer F.Cu) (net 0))
 (segment (start 110.18 82.82) (end 120.7 82.82) (width 0.5) (layer F.Cu) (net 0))
 (segment (start 108.2 84.8) (end 110.18 82.82) (width 0.5) (layer F.Cu) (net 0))
 (segment (start 125.05 103) (end 124.95 102.9) (width 0.5) (layer F.Cu) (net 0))
 (segment (start 126.8 103) (end 125.05 103) (width 0.5) (layer F.Cu) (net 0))
 (segment (start 124.95 102.9) (end 122 102.9) (width 0.5) (layer F.Cu) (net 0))
 (segment (start 120.7 104.2) (end 120.7 114.9) (width 0.5) (layer F.Cu) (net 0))
 (segment (start 122 102.9) (end 120.7 104.2) (width 0.5) (layer F.Cu) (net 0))
 (segment (start 87 122.063) (end 88.1 120.963) (width 0.5) (layer F.Cu) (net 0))
 (segment (start 84 122.063) (end 87 122.063) (width 0.5) (layer F.Cu) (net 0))
 (segment (start 88.1 120.963) (end 88.137 120.963) (width 0.5) (layer F.Cu) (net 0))
 (segment (start 88.137 120.963) (end 89.5 119.6) (width 0.5) (layer F.Cu) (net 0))
 (segment (start 89.5 119.6) (end 99.5 119.6) (width 0.5) (layer F.Cu) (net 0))
 (segment (start 101.963 122.063) (end 106 122.063) (width 0.5) (layer F.Cu) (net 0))
 (segment (start 99.5 119.6) (end 101.963 122.063) (width 0.5) (layer F.Cu) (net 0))
 (segment (start 87.037 68.861) (end 89.6 66.298) (width 0.5) (layer F.Cu) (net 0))
 (segment (start 84.037 68.861) (end 87.037 68.861) (width 0.5) (layer F.Cu) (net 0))
 (segment (start 89.6 66.298) (end 98.998 66.298) (width 0.5) (layer F.Cu) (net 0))
 (segment (start 101.561 68.861) (end 106.037 68.861) (width 0.5) (layer F.Cu) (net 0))
 (segment (start 98.998 66.298) (end 101.561 68.861) (width 0.5) (layer F.Cu) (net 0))
 (segment (start 122.55 61.6) (end 123.9 62.95) (width 0.5) (layer F.Cu) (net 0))
 (segment (start 120.8 61.6) (end 122.55 61.6) (width 0.5) (layer F.Cu) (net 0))
 (segment (start 123.9 62.95) (end 123.9 65.5) (width 0.5) (layer F.Cu) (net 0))
 (segment (start 124.2 65.8) (end 126.9 65.8) (width 0.5) (layer F.Cu) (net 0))
 (segment (start 123.9 65.5) (end 124.2 65.8) (width 0.5) (layer F.Cu) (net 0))
 (segment (start 113.6 58.6) (end 135.1 58.6) (width 0.5) (layer F.Cu) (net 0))
 (segment (start 104.9 60) (end 112.2 60) (width 0.5) (layer F.Cu) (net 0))
 (segment (start 112.2 60) (end 113.6 58.6) (width 0.5) (layer F.Cu) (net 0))
 (segment (start 165.6 88.6) (end 166.1 88.1) (width 0.5) (layer F.Cu) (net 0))
 (segment (start 165.6 94.3) (end 165.6 88.6) (width 0.5) (layer F.Cu) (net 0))
 (segment (start 167.421 110.388) (end 164.758 113.051) (width 0.5) (layer F.Cu) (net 2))
 (segment (start 167.421 109.388) (end 167.421 110.388) (width 0.5) (layer F.Cu) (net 2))
 (segment (start 164.742 114.198) (end 160.374 114.198) (width 0.5) (layer F.Cu) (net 2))
 (segment (start 164.758 114.214) (end 164.742 114.198) (width 0.5) (layer F.Cu) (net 2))
 (segment (start 164.758 113.051) (end 164.758 114.214) (width 0.5) (layer F.Cu) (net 2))
 (segment (start 167.421 108.388) (end 168.568 107.241) (width 0.5) (layer F.Cu) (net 2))
 (segment (start 167.421 109.388) (end 167.421 108.388) (width 0.5) (layer F.Cu) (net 2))
 (segment (start 170.731 103.563002) (end 170.731 102.768) (width 0.5) (layer F.Cu) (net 2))
 (segment (start 168.568 105.726002) (end 170.731 103.563002) (width 0.5) (layer F.Cu) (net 2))
 (segment (start 170.731 102.768) (end 170.731 101.768) (width 0.5) (layer F.Cu) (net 2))
 (segment (start 168.568 107.241) (end 168.568 105.726002) (width 0.5) (layer F.Cu) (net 2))
 (segment (start 135.6 123.8) (end 137.1 123.8) (width 0.5) (layer F.Cu) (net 2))
 (segment (start 157.371003 123.3) (end 157.371001 123.300002) (width 0.5) (layer F.Cu) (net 2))
 (segment (start 150.300999 123.300002) (end 150.300997 123.3) (width 0.5) (layer F.Cu) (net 2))
 (segment (start 152.291001 123.300002) (end 150.300999 123.300002) (width 0.5) (layer F.Cu) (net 2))
 (segment (start 164.758 114.214) (end 164.758 117.262) (width 0.5) (layer F.Cu) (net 2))
 (segment (start 158.72 123.3) (end 157.371003 123.3) (width 0.5) (layer F.Cu) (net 2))
 (segment (start 147.211003 123.3) (end 147.211001 123.300002) (width 0.5) (layer F.Cu) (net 2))
 (segment (start 164.758 117.262) (end 158.72 123.3) (width 0.5) (layer F.Cu) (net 2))
 (segment (start 155.380997 123.3) (end 152.291003 123.3) (width 0.5) (layer F.Cu) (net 2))
 (segment (start 152.291003 123.3) (end 152.291001 123.300002) (width 0.5) (layer F.Cu) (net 2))
 (segment (start 150.300997 123.3) (end 147.211003 123.3) (width 0.5) (layer F.Cu) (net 2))
 (segment (start 141.136 123.00999) (end 141.136 121.135) (width 0.5) (layer F.Cu) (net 2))
 (segment (start 147.211001 123.300002) (end 145.220999 123.300002) (width 0.5) (layer F.Cu) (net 2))
 (segment (start 157.371001 123.300002) (end 155.380999 123.300002) (width 0.5) (layer F.Cu) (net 2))
 (segment (start 145.220999 123.300002) (end 145.220997 123.3) (width 0.5) (layer F.Cu) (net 2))
 (segment (start 145.220997 123.3) (end 141.42601 123.3) (width 0.5) (layer F.Cu) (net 2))
 (segment (start 155.380999 123.300002) (end 155.380997 123.3) (width 0.5) (layer F.Cu) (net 2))
 (segment (start 141.42601 123.3) (end 141.136 123.00999) (width 0.5) (layer F.Cu) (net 2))
 (segment (start 135.6 117.9) (end 135.6 123.8) (width 0.5) (layer F.Cu) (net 2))
 (segment (start 141.136 121.135) (end 141.136 118.92) (width 0.5) (layer F.Cu) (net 2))
 (segment (start 141.1 118.884) (end 141.1 117.5) (width 0.5) (layer F.Cu) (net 2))
 (segment (start 137.5 116) (end 135.6 117.9) (width 0.5) (layer F.Cu) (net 2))
 (segment (start 141.136 118.92) (end 141.1 118.884) (width 0.5) (layer F.Cu) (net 2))
 (segment (start 141.1 117.5) (end 139.6 116) (width 0.5) (layer F.Cu) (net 2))
 (segment (start 139.6 116) (end 137.5 116) (width 0.5) (layer F.Cu) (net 2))
 (segment (start 170.731 112.928) (end 169.191 114.468) (width 0.5) (layer F.Cu) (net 9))
 (segment (start 170.731 111.928) (end 170.731 112.928) (width 0.5) (layer F.Cu) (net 9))
 (segment (start 169.191 114.468) (end 167.421 114.468) (width 0.5) (layer F.Cu) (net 9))
 (segment (start 167.421 115.468) (end 167.421 114.468) (width 0.5) (layer F.Cu) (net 9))
 (segment (start 167.421 115.588962) (end 167.421 115.468) (width 0.5) (layer F.Cu) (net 9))
 (segment (start 140.862 124.1) (end 158.909962 124.1) (width 0.5) (layer F.Cu) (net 9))
 (segment (start 158.909962 124.1) (end 167.421 115.588962) (width 0.5) (layer F.Cu) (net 9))
 (segment (start 138.596 118.215) (end 138.596 121.834) (width 0.5) (layer F.Cu) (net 9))
 (segment (start 138.596 121.834) (end 140.862 124.1) (width 0.5) (layer F.Cu) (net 9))
 (segment (start 156.138 114.198) (end 156.122 114.214) (width 0.5) (layer F.Cu) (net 10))
 (segment (start 158.474 114.198) (end 156.138 114.198) (width 0.5) (layer F.Cu) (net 10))
 (segment (start 167.421 106.217) (end 167.421 104.308) (width 0.5) (layer F.Cu) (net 10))
 (segment (start 160.340001 113.297999) (end 167.421 106.217) (width 0.5) (layer F.Cu) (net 10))
 (segment (start 158.474 114.198) (end 158.474 114.148) (width 0.5) (layer F.Cu) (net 10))
 (segment (start 159.324001 113.297999) (end 160.340001 113.297999) (width 0.5) (layer F.Cu) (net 10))
 (segment (start 158.474 114.148) (end 159.324001 113.297999) (width 0.5) (layer F.Cu) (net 10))
 (segment (start 153.836 114.223) (end 153.836 118.215) (width 0.5) (layer F.Cu) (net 8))
 (segment (start 153.836 113.648) (end 154.286 113.198) (width 0.25) (layer F.Cu) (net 8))
 (segment (start 153.836 114.223) (end 153.836 113.648) (width 0.25) (layer F.Cu) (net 8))
 (segment (start 159.424 112.248) (end 159.424 112.198) (width 0.25) (layer F.Cu) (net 8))
 (segment (start 158.474 113.198) (end 159.424 112.248) (width 0.25) (layer F.Cu) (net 8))
 (segment (start 154.286 113.198) (end 158.474 113.198) (width 0.25) (layer F.Cu) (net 8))
 (segment (start 153.845 112.164) (end 153.836 112.173) (width 0.5) (layer F.Cu) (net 7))
 (segment (start 156.122 112.164) (end 153.845 112.164) (width 0.5) (layer F.Cu) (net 7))
 (segment (start 153.136 112.173) (end 153.836 112.173) (width 0.5) (layer F.Cu) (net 7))
 (segment (start 151.972997 112.173) (end 153.136 112.173) (width 0.5) (layer F.Cu) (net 7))
 (segment (start 138.64 98.840003) (end 151.972997 112.173) (width 0.5) (layer F.Cu) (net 7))
 (segment (start 138.64 95.3) (end 138.64 98.840003) (width 0.5) (layer F.Cu) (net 7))
 (segment (start 148.756 116) (end 148.756 118.215) (width 0.5) (layer F.Cu) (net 1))
 (segment (start 148.056 115.3) (end 148.756 116) (width 0.5) (layer F.Cu) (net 1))
 (segment (start 137.1 115.3) (end 148.056 115.3) (width 0.5) (layer F.Cu) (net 1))
 (segment (start 126.8 117.5) (end 134.9 117.5) (width 0.5) (layer F.Cu) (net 1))
 (segment (start 134.9 117.5) (end 137.1 115.3) (width 0.5) (layer F.Cu) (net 1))
 (segment (start 82.8 45.5) (end 88.6 45.5) (width 0.5) (layer F.Cu) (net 6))
 (segment (start 90.625 47.525) (end 98.8 47.525) (width 0.5) (layer F.Cu) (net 6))
 (segment (start 88.6 45.5) (end 90.625 47.525) (width 0.5) (layer F.Cu) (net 6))
 (segment (start 91.4 114.9) (end 98.7 114.9) (width 0.5) (layer F.Cu) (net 5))
 (segment (start 82.875 113.4) (end 89.9 113.4) (width 0.5) (layer F.Cu) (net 5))
 (segment (start 89.9 113.4) (end 91.4 114.9) (width 0.5) (layer F.Cu) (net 5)))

